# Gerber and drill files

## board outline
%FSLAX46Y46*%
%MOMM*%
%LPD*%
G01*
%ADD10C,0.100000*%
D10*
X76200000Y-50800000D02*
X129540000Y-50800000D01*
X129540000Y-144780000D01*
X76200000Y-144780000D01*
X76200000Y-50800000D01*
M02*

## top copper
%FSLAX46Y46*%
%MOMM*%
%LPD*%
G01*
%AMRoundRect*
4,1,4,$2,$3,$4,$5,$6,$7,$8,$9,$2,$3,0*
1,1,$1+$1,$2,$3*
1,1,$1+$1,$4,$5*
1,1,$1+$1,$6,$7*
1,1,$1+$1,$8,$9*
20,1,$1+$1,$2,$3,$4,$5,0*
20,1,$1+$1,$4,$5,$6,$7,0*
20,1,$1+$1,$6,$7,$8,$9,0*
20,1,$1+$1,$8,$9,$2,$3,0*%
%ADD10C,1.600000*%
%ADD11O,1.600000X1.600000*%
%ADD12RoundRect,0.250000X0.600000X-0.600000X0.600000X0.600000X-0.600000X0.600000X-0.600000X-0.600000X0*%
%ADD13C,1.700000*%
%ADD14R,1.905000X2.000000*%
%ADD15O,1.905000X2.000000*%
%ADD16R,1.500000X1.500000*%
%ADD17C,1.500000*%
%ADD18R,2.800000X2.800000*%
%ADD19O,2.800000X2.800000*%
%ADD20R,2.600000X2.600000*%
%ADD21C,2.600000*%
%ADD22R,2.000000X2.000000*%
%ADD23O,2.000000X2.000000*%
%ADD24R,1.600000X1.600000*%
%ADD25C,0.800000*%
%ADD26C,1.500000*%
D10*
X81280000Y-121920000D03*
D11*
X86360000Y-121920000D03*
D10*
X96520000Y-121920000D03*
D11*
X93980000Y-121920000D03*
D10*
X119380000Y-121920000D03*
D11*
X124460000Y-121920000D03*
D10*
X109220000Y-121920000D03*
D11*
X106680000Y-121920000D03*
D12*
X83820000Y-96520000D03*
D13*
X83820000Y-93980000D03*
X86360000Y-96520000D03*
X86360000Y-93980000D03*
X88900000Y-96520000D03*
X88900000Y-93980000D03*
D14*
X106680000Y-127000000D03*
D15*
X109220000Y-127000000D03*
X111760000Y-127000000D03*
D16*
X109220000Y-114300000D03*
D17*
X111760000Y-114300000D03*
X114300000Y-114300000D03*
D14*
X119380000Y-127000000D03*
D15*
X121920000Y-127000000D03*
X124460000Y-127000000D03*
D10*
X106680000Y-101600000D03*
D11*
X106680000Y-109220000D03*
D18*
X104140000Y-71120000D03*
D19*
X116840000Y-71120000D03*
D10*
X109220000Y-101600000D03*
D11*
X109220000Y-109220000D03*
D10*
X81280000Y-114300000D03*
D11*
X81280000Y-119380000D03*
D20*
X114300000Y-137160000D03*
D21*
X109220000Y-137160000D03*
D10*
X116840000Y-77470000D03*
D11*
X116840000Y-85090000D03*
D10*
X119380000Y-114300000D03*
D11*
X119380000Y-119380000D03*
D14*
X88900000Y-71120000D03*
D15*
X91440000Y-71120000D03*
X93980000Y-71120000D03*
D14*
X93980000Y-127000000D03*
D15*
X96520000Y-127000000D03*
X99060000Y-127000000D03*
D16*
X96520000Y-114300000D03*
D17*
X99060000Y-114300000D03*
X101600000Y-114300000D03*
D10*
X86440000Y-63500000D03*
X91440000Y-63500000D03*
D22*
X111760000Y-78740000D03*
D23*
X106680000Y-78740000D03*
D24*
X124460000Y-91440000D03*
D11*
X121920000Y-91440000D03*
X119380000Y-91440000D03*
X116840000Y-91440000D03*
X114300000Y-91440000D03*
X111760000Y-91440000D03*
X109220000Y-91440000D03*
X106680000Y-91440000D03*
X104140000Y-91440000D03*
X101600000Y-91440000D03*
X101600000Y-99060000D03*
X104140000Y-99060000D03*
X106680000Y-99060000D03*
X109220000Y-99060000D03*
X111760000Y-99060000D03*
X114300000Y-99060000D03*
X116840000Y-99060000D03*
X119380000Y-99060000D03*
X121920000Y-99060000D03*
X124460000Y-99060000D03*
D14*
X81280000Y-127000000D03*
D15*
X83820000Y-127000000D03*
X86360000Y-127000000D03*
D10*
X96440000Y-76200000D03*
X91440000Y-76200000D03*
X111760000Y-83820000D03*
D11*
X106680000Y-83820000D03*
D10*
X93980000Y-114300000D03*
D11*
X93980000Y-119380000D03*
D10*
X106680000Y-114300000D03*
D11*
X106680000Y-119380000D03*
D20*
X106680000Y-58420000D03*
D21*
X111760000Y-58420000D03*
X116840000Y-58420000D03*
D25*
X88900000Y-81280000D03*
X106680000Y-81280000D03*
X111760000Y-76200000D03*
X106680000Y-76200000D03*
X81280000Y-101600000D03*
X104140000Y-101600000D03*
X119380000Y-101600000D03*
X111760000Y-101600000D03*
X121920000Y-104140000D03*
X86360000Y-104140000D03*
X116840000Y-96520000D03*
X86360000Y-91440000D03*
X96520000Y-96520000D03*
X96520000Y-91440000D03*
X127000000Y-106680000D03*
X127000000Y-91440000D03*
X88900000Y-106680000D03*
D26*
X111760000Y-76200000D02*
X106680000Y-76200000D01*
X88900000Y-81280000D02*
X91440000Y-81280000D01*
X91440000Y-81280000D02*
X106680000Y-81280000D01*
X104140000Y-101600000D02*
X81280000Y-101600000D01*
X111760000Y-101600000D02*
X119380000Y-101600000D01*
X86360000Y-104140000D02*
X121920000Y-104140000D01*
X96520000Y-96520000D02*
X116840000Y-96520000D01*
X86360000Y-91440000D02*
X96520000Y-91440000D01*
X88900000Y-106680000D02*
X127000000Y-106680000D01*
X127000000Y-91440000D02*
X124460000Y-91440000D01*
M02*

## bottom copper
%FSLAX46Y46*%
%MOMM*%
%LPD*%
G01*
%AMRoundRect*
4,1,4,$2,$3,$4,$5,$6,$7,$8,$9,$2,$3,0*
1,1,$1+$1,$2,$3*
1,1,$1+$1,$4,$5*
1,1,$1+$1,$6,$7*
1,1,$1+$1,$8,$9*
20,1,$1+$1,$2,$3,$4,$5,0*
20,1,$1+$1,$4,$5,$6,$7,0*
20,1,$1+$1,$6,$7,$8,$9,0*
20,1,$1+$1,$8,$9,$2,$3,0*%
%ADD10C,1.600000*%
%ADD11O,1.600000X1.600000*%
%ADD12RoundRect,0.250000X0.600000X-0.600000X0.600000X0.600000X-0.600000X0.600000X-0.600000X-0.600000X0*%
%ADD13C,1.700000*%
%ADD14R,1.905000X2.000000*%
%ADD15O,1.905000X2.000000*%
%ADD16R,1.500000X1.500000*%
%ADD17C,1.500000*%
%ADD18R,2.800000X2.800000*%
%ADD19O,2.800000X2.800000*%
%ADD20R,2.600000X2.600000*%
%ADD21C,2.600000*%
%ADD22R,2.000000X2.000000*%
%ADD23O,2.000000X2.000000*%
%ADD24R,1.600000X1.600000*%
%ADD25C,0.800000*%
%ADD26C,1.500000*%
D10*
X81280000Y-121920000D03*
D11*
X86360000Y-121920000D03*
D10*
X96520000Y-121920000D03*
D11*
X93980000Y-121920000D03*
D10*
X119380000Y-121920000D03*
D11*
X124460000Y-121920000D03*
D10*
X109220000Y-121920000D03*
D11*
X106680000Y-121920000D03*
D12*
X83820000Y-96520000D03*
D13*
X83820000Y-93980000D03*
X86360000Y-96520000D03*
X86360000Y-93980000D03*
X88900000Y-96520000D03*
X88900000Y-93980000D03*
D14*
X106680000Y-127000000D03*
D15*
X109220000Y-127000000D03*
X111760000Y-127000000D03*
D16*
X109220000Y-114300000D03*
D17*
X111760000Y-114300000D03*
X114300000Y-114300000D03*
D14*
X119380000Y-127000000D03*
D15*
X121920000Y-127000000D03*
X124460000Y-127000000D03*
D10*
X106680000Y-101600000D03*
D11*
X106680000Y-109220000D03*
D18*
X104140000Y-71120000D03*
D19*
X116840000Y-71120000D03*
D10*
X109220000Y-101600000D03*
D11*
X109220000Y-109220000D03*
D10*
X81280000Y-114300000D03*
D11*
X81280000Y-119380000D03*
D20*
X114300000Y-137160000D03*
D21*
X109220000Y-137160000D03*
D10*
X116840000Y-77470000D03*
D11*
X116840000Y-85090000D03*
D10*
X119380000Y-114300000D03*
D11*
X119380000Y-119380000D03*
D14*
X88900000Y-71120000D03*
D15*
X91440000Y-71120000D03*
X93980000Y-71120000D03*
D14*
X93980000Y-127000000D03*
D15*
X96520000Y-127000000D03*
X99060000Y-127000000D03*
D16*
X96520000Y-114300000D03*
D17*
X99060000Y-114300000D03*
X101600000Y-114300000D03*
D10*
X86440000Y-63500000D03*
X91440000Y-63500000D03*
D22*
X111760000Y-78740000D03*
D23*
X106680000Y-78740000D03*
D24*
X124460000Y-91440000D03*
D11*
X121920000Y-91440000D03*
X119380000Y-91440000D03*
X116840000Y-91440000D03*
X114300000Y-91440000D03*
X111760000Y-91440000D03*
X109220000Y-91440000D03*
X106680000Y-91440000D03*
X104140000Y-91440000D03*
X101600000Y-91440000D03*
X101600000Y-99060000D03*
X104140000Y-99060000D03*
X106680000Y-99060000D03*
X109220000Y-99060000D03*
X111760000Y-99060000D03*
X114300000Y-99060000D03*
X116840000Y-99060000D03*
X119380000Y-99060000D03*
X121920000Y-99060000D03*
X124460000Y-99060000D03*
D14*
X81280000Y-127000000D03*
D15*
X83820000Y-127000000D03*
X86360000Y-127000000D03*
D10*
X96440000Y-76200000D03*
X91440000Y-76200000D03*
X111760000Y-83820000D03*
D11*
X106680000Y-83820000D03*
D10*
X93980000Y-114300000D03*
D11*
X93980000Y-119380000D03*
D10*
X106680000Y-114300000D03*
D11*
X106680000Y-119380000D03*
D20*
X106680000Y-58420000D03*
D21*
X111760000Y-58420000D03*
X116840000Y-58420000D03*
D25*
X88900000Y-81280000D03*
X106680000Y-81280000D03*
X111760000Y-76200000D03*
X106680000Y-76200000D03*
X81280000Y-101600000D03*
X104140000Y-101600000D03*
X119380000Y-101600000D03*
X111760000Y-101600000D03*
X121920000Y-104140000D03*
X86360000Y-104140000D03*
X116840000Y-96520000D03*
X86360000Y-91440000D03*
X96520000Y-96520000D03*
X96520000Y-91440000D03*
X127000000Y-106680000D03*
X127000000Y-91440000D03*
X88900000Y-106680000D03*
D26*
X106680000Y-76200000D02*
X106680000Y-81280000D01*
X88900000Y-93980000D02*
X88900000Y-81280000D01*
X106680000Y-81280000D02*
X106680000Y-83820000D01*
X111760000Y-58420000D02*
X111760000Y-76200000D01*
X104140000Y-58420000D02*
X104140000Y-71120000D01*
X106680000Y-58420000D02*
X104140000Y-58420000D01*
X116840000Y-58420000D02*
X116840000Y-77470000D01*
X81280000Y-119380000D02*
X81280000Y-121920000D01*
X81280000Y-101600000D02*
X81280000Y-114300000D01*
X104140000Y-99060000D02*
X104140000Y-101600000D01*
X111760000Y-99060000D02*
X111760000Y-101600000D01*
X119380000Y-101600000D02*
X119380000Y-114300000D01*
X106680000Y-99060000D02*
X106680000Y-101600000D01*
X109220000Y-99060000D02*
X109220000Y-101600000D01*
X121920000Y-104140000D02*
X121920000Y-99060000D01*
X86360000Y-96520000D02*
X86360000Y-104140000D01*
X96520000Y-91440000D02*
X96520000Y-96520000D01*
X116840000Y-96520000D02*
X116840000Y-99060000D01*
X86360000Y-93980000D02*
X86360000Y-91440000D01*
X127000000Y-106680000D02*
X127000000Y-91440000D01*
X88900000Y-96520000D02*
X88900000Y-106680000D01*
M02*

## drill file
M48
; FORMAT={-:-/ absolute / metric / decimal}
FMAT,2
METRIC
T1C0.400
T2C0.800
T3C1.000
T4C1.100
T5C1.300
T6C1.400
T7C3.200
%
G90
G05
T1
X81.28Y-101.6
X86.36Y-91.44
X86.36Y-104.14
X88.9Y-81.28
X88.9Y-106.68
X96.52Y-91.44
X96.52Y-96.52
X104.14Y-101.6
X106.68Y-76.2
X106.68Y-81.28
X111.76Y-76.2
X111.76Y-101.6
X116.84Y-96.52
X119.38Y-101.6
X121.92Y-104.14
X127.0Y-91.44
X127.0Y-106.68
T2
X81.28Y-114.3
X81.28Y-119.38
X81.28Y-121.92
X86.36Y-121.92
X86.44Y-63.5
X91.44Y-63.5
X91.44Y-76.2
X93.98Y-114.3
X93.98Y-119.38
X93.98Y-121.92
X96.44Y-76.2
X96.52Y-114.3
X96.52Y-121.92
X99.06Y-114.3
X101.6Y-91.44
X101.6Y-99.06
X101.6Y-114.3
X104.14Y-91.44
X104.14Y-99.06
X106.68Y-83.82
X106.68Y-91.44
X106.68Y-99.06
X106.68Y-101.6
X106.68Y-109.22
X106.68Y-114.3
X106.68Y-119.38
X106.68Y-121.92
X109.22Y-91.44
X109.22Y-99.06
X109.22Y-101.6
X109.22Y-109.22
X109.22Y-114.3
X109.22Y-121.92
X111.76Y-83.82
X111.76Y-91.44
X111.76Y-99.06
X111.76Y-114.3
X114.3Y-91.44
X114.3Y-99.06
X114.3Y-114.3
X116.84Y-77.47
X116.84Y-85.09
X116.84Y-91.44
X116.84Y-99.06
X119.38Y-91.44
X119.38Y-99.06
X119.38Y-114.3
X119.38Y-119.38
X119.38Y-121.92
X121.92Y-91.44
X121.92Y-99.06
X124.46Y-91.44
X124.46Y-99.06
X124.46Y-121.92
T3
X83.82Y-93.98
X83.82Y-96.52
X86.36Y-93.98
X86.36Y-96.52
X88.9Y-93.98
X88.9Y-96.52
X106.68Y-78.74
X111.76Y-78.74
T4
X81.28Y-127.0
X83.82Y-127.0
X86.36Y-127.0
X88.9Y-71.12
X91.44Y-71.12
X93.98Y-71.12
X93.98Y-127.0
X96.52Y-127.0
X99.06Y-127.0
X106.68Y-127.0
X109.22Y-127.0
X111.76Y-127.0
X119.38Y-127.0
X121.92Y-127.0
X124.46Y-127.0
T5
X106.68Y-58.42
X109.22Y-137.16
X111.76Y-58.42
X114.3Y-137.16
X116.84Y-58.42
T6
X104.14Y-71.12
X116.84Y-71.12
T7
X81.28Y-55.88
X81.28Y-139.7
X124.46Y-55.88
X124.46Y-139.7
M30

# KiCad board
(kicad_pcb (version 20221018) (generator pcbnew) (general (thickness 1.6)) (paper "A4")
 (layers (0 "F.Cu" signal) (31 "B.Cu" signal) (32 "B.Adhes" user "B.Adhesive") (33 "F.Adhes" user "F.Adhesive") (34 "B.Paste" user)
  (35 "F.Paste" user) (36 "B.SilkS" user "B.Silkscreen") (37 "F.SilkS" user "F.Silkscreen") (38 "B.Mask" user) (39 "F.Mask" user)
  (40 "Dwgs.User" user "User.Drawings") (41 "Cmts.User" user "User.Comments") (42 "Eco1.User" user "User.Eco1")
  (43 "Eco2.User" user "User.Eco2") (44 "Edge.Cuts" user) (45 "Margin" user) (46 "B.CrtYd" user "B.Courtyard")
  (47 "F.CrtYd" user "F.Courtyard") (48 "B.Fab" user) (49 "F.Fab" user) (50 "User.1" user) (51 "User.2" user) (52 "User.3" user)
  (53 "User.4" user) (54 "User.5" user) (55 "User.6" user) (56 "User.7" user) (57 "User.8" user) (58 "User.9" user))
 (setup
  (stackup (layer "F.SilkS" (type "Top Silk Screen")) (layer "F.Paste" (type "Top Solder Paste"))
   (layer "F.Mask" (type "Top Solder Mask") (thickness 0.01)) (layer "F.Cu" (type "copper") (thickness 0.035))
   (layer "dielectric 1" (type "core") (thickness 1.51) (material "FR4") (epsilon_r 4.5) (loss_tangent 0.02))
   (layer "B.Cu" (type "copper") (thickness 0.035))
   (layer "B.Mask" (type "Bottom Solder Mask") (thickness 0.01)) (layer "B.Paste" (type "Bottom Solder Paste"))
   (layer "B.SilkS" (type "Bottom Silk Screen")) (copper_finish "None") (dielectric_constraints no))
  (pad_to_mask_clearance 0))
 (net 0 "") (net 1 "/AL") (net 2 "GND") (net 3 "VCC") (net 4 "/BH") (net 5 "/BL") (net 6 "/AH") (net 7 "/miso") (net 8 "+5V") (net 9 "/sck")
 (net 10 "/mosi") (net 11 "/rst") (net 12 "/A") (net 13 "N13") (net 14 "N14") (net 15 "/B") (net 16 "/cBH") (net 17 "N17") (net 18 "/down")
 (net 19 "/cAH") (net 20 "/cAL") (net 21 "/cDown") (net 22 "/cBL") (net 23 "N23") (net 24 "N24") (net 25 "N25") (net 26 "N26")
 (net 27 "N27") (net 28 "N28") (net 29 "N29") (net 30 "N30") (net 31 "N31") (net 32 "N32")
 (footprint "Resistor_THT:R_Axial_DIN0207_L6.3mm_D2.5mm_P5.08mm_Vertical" (layer "F.Cu") (at 81.28 121.92)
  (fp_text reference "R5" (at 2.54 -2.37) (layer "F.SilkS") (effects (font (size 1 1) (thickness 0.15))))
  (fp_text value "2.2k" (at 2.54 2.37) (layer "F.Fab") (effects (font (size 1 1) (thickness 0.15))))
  (pad "1" thru_hole circle (at 0 0) (size 1.6 1.6) (drill 0.8) (layers "*.Cu" "*.Mask") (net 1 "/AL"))
  (pad "2" thru_hole oval (at 5.08 0) (size 1.6 1.6) (drill 0.8) (layers "*.Cu" "*.Mask") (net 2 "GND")))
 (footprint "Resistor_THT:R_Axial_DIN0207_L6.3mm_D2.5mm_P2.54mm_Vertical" (layer "F.Cu") (at 96.52 121.92 180)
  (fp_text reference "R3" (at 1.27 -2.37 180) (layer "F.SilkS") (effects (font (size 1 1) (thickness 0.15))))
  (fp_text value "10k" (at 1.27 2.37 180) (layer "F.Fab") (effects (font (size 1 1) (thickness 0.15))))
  (pad "1" thru_hole circle (at 0 0 180) (size 1.6 1.6) (drill 0.8) (layers "*.Cu" "*.Mask") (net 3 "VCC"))
  (pad "2" thru_hole oval (at 2.54 0 180) (size 1.6 1.6) (drill 0.8) (layers "*.Cu" "*.Mask") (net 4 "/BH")))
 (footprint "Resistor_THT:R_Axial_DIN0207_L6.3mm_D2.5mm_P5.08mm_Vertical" (layer "F.Cu") (at 119.38 121.92)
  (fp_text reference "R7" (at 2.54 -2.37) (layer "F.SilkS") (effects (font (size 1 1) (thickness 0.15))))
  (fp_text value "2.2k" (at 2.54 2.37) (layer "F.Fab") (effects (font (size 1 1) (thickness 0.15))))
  (pad "1" thru_hole circle (at 0 0) (size 1.6 1.6) (drill 0.8) (layers "*.Cu" "*.Mask") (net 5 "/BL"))
  (pad "2" thru_hole oval (at 5.08 0) (size 1.6 1.6) (drill 0.8) (layers "*.Cu" "*.Mask") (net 2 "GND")))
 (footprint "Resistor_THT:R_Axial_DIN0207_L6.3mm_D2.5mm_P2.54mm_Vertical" (layer "F.Cu") (at 109.22 121.92 180)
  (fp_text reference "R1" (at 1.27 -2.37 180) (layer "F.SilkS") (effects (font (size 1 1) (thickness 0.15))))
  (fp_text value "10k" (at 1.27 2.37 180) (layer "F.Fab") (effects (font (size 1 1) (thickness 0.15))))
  (pad "1" thru_hole circle (at 0 0 180) (size 1.6 1.6) (drill 0.8) (layers "*.Cu" "*.Mask") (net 3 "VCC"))
  (pad "2" thru_hole oval (at 2.54 0 180) (size 1.6 1.6) (drill 0.8) (layers "*.Cu" "*.Mask") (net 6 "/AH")))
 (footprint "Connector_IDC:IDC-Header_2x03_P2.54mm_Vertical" (layer "F.Cu") (at 83.82 96.52 90)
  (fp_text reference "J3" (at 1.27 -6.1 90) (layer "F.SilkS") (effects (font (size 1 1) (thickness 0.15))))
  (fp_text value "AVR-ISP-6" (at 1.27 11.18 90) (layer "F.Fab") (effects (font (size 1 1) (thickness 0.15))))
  (pad "1" thru_hole roundrect (at 0 0 90) (size 1.7 1.7) (drill 1) (layers "*.Cu" "*.Mask") (roundrect_rratio 0.147059) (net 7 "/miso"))
  (pad "2" thru_hole circle (at 2.54 0 90) (size 1.7 1.7) (drill 1) (layers "*.Cu" "*.Mask") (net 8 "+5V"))
  (pad "3" thru_hole circle (at 0 2.54 90) (size 1.7 1.7) (drill 1) (layers "*.Cu" "*.Mask") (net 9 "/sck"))
  (pad "4" thru_hole circle (at 2.54 2.54 90) (size 1.7 1.7) (drill 1) (layers "*.Cu" "*.Mask") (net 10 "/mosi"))
  (pad "5" thru_hole circle (at 0 5.08 90) (size 1.7 1.7) (drill 1) (layers "*.Cu" "*.Mask") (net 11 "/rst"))
  (pad "6" thru_hole circle (at 2.54 5.08 90) (size 1.7 1.7) (drill 1) (layers "*.Cu" "*.Mask") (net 2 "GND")))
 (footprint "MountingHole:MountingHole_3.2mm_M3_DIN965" (layer "F.Cu") (at 81.28 139.7)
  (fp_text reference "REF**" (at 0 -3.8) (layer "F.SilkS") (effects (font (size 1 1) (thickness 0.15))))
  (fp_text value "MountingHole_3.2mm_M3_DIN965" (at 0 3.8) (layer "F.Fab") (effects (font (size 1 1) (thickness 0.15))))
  (pad "" np_thru_hole circle (at 0 0) (size 3.2 3.2) (drill 3.2) (layers "*.Cu" "*.Mask")))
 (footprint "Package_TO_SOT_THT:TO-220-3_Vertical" (layer "F.Cu") (at 106.68 127)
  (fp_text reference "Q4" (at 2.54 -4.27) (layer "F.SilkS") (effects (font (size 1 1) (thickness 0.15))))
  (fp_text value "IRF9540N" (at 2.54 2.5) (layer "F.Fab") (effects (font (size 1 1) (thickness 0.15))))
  (pad "1" thru_hole rect (at 0 0) (size 1.905 2) (drill 1.1) (layers "*.Cu" "*.Mask") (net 6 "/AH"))
  (pad "2" thru_hole oval (at 2.54 0) (size 1.905 2) (drill 1.1) (layers "*.Cu" "*.Mask") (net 3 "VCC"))
  (pad "3" thru_hole oval (at 5.08 0) (size 1.905 2) (drill 1.1) (layers "*.Cu" "*.Mask") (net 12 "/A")))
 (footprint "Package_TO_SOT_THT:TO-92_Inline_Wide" (layer "F.Cu") (at 109.22 114.3)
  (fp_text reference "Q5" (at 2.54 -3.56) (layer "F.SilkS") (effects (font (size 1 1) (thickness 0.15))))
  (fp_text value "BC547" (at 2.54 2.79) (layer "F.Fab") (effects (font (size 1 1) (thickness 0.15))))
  (pad "1" thru_hole rect (at 0 0) (size 1.5 1.5) (drill 0.8) (layers "*.Cu" "*.Mask") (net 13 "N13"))
  (pad "2" thru_hole circle (at 2.54 0) (size 1.5 1.5) (drill 0.8) (layers "*.Cu" "*.Mask") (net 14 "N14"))
  (pad "3" thru_hole circle (at 5.08 0) (size 1.5 1.5) (drill 0.8) (layers "*.Cu" "*.Mask") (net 2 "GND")))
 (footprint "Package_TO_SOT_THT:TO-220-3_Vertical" (layer "F.Cu") (at 119.38 127)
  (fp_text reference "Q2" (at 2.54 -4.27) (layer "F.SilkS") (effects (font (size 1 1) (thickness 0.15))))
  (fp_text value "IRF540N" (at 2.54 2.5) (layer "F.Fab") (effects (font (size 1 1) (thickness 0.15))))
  (pad "1" thru_hole rect (at 0 0) (size 1.905 2) (drill 1.1) (layers "*.Cu" "*.Mask") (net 5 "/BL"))
  (pad "2" thru_hole oval (at 2.54 0) (size 1.905 2) (drill 1.1) (layers "*.Cu" "*.Mask") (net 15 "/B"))
  (pad "3" thru_hole oval (at 5.08 0) (size 1.905 2) (drill 1.1) (layers "*.Cu" "*.Mask") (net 2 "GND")))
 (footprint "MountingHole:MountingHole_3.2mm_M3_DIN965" (layer "F.Cu") (at 124.46 55.88)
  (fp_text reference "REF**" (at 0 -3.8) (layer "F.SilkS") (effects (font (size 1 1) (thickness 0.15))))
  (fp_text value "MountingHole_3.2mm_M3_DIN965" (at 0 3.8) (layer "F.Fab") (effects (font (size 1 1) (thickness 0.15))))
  (pad "" np_thru_hole circle (at 0 0) (size 3.2 3.2) (drill 3.2) (layers "*.Cu" "*.Mask")))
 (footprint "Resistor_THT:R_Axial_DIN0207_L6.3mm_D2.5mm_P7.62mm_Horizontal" (layer "F.Cu") (at 106.68 101.6 -90)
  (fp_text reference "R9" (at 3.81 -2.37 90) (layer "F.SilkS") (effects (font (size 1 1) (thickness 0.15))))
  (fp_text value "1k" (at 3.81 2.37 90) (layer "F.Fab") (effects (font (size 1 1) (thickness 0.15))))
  (pad "1" thru_hole circle (at 0 0 270) (size 1.6 1.6) (drill 0.8) (layers "*.Cu" "*.Mask") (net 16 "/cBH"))
  (pad "2" thru_hole oval (at 7.62 0 270) (size 1.6 1.6) (drill 0.8) (layers "*.Cu" "*.Mask") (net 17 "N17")))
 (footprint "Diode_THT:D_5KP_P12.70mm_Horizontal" (layer "F.Cu") (at 104.14 71.12)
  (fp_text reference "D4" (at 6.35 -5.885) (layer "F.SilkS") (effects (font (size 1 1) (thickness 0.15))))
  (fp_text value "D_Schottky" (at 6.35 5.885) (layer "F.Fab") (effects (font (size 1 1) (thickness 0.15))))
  (pad "1" thru_hole rect (at 0 0) (size 2.8 2.8) (drill 1.4) (layers "*.Cu" "*.Mask") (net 3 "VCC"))
  (pad "2" thru_hole oval (at 12.7 0) (size 2.8 2.8) (drill 1.4) (layers "*.Cu" "*.Mask") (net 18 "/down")))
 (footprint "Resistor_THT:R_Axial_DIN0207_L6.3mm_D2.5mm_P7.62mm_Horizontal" (layer "F.Cu") (at 109.22 101.6 -90)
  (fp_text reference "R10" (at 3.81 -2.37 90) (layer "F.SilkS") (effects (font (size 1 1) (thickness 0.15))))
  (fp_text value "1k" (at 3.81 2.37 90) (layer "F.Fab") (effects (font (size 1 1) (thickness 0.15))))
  (pad "1" thru_hole circle (at 0 0 270) (size 1.6 1.6) (drill 0.8) (layers "*.Cu" "*.Mask") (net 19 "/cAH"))
  (pad "2" thru_hole oval (at 7.62 0 270) (size 1.6 1.6) (drill 0.8) (layers "*.Cu" "*.Mask") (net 14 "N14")))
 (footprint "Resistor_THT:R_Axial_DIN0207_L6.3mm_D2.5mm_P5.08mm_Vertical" (layer "F.Cu") (at 81.28 114.3 -90)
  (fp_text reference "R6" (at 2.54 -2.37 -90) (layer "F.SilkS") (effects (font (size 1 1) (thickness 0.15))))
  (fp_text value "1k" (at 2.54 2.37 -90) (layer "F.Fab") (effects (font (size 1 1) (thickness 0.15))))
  (pad "1" thru_hole circle (at 0 0 270) (size 1.6 1.6) (drill 0.8) (layers "*.Cu" "*.Mask") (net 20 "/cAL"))
  (pad "2" thru_hole oval (at 5.08 0 270) (size 1.6 1.6) (drill 0.8) (layers "*.Cu" "*.Mask") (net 1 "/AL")))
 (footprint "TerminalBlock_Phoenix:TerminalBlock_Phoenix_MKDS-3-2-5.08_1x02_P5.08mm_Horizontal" (layer "F.Cu") (at 114.3 137.16 180)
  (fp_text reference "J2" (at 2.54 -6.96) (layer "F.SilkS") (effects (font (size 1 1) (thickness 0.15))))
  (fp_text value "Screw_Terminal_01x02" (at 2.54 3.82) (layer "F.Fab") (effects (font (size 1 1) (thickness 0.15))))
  (pad "1" thru_hole rect (at 0 0 180) (size 2.6 2.6) (drill 1.3) (layers "*.Cu" "*.Mask") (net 12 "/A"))
  (pad "2" thru_hole circle (at 5.08 0 180) (size 2.6 2.6) (drill 1.3) (layers "*.Cu" "*.Mask") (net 15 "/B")))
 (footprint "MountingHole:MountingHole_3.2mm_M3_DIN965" (layer "F.Cu") (at 124.46 139.7)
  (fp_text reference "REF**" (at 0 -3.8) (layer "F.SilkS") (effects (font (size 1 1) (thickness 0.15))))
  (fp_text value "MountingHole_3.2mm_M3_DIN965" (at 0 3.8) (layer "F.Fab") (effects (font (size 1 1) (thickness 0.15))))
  (pad "" np_thru_hole circle (at 0 0) (size 3.2 3.2) (drill 3.2) (layers "*.Cu" "*.Mask")))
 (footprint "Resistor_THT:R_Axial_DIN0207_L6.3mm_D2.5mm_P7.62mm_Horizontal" (layer "F.Cu") (at 116.84 77.47 -90)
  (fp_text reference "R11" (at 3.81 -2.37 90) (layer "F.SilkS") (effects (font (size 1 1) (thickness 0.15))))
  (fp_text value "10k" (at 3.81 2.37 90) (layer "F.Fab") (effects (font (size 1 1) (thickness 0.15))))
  (pad "1" thru_hole circle (at 0 0 270) (size 1.6 1.6) (drill 0.8) (layers "*.Cu" "*.Mask") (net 18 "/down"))
  (pad "2" thru_hole oval (at 7.62 0 270) (size 1.6 1.6) (drill 0.8) (layers "*.Cu" "*.Mask") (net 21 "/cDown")))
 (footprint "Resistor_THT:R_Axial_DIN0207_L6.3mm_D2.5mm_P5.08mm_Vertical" (layer "F.Cu") (at 119.38 114.3 -90)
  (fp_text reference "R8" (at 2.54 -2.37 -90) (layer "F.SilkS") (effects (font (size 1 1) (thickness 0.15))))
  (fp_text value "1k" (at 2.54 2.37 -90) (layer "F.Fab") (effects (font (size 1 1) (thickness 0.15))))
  (pad "1" thru_hole circle (at 0 0 270) (size 1.6 1.6) (drill 0.8) (layers "*.Cu" "*.Mask") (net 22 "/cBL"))
  (pad "2" thru_hole oval (at 5.08 0 270) (size 1.6 1.6) (drill 0.8) (layers "*.Cu" "*.Mask") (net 5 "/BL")))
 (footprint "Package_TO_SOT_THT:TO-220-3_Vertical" (layer "F.Cu") (at 88.9 71.12)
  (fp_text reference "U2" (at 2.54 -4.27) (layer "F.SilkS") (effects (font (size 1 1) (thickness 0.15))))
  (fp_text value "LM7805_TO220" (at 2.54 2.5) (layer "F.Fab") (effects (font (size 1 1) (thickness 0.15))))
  (pad "1" thru_hole rect (at 0 0) (size 1.905 2) (drill 1.1) (layers "*.Cu" "*.Mask") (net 3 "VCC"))
  (pad "2" thru_hole oval (at 2.54 0) (size 1.905 2) (drill 1.1) (layers "*.Cu" "*.Mask") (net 2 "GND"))
  (pad "3" thru_hole oval (at 5.08 0) (size 1.905 2) (drill 1.1) (layers "*.Cu" "*.Mask") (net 8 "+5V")))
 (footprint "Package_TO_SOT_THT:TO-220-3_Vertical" (layer "F.Cu") (at 93.98 127)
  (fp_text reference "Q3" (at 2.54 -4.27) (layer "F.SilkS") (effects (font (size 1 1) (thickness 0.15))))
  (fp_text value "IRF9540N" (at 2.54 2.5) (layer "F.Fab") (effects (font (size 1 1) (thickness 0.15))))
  (pad "1" thru_hole rect (at 0 0) (size 1.905 2) (drill 1.1) (layers "*.Cu" "*.Mask") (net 4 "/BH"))
  (pad "2" thru_hole oval (at 2.54 0) (size 1.905 2) (drill 1.1) (layers "*.Cu" "*.Mask") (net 3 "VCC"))
  (pad "3" thru_hole oval (at 5.08 0) (size 1.905 2) (drill 1.1) (layers "*.Cu" "*.Mask") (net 15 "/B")))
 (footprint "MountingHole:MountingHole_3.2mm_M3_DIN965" (layer "F.Cu") (at 81.28 55.88)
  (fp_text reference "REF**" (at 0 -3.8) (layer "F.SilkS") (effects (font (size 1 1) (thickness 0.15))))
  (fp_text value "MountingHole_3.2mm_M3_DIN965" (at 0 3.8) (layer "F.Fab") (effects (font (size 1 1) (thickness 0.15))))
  (pad "" np_thru_hole circle (at 0 0) (size 3.2 3.2) (drill 3.2) (layers "*.Cu" "*.Mask")))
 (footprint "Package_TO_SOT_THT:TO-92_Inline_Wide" (layer "F.Cu") (at 96.52 114.3)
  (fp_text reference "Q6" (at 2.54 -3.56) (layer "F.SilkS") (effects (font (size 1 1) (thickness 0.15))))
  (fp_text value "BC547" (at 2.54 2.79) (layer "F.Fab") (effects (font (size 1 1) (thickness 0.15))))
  (pad "1" thru_hole rect (at 0 0) (size 1.5 1.5) (drill 0.8) (layers "*.Cu" "*.Mask") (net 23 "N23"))
  (pad "2" thru_hole circle (at 2.54 0) (size 1.5 1.5) (drill 0.8) (layers "*.Cu" "*.Mask") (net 17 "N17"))
  (pad "3" thru_hole circle (at 5.08 0) (size 1.5 1.5) (drill 0.8) (layers "*.Cu" "*.Mask") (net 2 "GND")))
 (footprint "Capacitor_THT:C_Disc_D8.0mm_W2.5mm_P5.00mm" (layer "F.Cu") (at 86.44 63.5)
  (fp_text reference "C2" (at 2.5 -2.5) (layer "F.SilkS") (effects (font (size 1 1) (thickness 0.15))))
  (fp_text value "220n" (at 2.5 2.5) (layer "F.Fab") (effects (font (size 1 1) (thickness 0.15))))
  (pad "1" thru_hole circle (at 0 0) (size 1.6 1.6) (drill 0.8) (layers "*.Cu" "*.Mask") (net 3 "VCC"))
  (pad "2" thru_hole circle (at 5 0) (size 1.6 1.6) (drill 0.8) (layers "*.Cu" "*.Mask") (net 2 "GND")))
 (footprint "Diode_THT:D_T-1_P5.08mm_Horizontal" (layer "F.Cu") (at 111.76 78.74 180)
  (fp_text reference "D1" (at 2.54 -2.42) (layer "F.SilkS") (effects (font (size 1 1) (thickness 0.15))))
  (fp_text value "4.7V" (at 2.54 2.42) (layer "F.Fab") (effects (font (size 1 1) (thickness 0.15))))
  (pad "1" thru_hole rect (at 0 0 180) (size 2 2) (drill 1) (layers "*.Cu" "*.Mask") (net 21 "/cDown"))
  (pad "2" thru_hole oval (at 5.08 0 180) (size 2 2) (drill 1) (layers "*.Cu" "*.Mask") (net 2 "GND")))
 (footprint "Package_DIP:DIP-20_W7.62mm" (layer "F.Cu") (at 124.46 91.44 -90)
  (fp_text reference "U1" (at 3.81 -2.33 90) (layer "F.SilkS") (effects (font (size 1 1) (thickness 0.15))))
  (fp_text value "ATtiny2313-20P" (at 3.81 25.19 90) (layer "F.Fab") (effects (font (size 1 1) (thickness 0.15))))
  (pad "1" thru_hole rect (at 0 0 270) (size 1.6 1.6) (drill 0.8) (layers "*.Cu" "*.Mask") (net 11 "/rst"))
  (pad "2" thru_hole oval (at 0 2.54 270) (size 1.6 1.6) (drill 0.8) (layers "*.Cu" "*.Mask") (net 21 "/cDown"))
  (pad "3" thru_hole oval (at 0 5.08 270) (size 1.6 1.6) (drill 0.8) (layers "*.Cu" "*.Mask") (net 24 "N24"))
  (pad "4" thru_hole oval (at 0 7.62 270) (size 1.6 1.6) (drill 0.8) (layers "*.Cu" "*.Mask") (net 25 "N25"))
  (pad "5" thru_hole oval (at 0 10.16 270) (size 1.6 1.6) (drill 0.8) (layers "*.Cu" "*.Mask") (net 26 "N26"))
  (pad "6" thru_hole oval (at 0 12.7 270) (size 1.6 1.6) (drill 0.8) (layers "*.Cu" "*.Mask") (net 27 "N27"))
  (pad "7" thru_hole oval (at 0 15.24 270) (size 1.6 1.6) (drill 0.8) (layers "*.Cu" "*.Mask") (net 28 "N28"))
  (pad "8" thru_hole oval (at 0 17.78 270) (size 1.6 1.6) (drill 0.8) (layers "*.Cu" "*.Mask") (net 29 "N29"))
  (pad "9" thru_hole oval (at 0 20.32 270) (size 1.6 1.6) (drill 0.8) (layers "*.Cu" "*.Mask") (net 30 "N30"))
  (pad "10" thru_hole oval (at 0 22.86 270) (size 1.6 1.6) (drill 0.8) (layers "*.Cu" "*.Mask") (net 2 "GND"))
  (pad "11" thru_hole oval (at 7.62 22.86 270) (size 1.6 1.6) (drill 0.8) (layers "*.Cu" "*.Mask") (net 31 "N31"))
  (pad "12" thru_hole oval (at 7.62 20.32 270) (size 1.6 1.6) (drill 0.8) (layers "*.Cu" "*.Mask") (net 20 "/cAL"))
  (pad "13" thru_hole oval (at 7.62 17.78 270) (size 1.6 1.6) (drill 0.8) (layers "*.Cu" "*.Mask") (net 16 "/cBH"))
  (pad "14" thru_hole oval (at 7.62 15.24 270) (size 1.6 1.6) (drill 0.8) (layers "*.Cu" "*.Mask") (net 19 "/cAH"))
  (pad "15" thru_hole oval (at 7.62 12.7 270) (size 1.6 1.6) (drill 0.8) (layers "*.Cu" "*.Mask") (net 22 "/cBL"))
  (pad "16" thru_hole oval (at 7.62 10.16 270) (size 1.6 1.6) (drill 0.8) (layers "*.Cu" "*.Mask") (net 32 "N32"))
  (pad "17" thru_hole oval (at 7.62 7.62 270) (size 1.6 1.6) (drill 0.8) (layers "*.Cu" "*.Mask") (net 10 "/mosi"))
  (pad "18" thru_hole oval (at 7.62 5.08 270) (size 1.6 1.6) (drill 0.8) (layers "*.Cu" "*.Mask") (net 7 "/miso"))
  (pad "19" thru_hole oval (at 7.62 2.54 270) (size 1.6 1.6) (drill 0.8) (layers "*.Cu" "*.Mask") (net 9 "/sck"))
  (pad "20" thru_hole oval (at 7.62 0 270) (size 1.6 1.6) (drill 0.8) (layers "*.Cu" "*.Mask") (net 8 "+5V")))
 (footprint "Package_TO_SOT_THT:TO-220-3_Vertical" (layer "F.Cu") (at 81.28 127)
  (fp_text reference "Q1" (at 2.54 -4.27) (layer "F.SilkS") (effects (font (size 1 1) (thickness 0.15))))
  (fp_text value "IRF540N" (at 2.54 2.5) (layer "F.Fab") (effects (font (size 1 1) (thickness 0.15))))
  (pad "1" thru_hole rect (at 0 0) (size 1.905 2) (drill 1.1) (layers "*.Cu" "*.Mask") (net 1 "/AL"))
  (pad "2" thru_hole oval (at 2.54 0) (size 1.905 2) (drill 1.1) (layers "*.Cu" "*.Mask") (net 12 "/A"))
  (pad "3" thru_hole oval (at 5.08 0) (size 1.905 2) (drill 1.1) (layers "*.Cu" "*.Mask") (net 2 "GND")))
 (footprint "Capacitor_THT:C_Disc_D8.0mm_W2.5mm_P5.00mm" (layer "F.Cu") (at 96.44 76.2 180)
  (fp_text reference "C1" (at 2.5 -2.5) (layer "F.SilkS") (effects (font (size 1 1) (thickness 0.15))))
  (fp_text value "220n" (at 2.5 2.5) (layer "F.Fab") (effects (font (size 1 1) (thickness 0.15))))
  (pad "1" thru_hole circle (at 0 0 180) (size 1.6 1.6) (drill 0.8) (layers "*.Cu" "*.Mask") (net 8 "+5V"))
  (pad "2" thru_hole circle (at 5 0 180) (size 1.6 1.6) (drill 0.8) (layers "*.Cu" "*.Mask") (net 2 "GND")))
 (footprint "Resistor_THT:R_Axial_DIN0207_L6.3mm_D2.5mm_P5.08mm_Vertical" (layer "F.Cu") (at 111.76 83.82 180)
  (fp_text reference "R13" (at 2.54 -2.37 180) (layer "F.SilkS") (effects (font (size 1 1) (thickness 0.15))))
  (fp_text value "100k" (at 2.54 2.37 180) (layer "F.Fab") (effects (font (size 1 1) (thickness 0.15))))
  (pad "1" thru_hole circle (at 0 0 180) (size 1.6 1.6) (drill 0.8) (layers "*.Cu" "*.Mask") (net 21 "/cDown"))
  (pad "2" thru_hole oval (at 5.08 0 180) (size 1.6 1.6) (drill 0.8) (layers "*.Cu" "*.Mask") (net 2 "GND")))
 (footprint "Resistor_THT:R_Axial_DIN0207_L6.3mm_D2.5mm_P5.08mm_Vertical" (layer "F.Cu") (at 93.98 114.3 -90)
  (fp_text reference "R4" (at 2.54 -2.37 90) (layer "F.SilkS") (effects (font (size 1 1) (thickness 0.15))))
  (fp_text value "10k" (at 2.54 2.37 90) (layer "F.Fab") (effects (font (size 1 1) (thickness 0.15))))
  (pad "1" thru_hole circle (at 0 0 270) (size 1.6 1.6) (drill 0.8) (layers "*.Cu" "*.Mask") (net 23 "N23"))
  (pad "2" thru_hole oval (at 5.08 0 270) (size 1.6 1.6) (drill 0.8) (layers "*.Cu" "*.Mask") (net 4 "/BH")))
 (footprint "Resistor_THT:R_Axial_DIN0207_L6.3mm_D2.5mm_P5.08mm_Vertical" (layer "F.Cu") (at 106.68 114.3 -90)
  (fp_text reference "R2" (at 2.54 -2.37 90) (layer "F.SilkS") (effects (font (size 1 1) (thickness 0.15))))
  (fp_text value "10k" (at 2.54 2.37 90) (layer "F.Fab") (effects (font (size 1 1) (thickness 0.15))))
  (pad "1" thru_hole circle (at 0 0 270) (size 1.6 1.6) (drill 0.8) (layers "*.Cu" "*.Mask") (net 13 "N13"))
  (pad "2" thru_hole oval (at 5.08 0 270) (size 1.6 1.6) (drill 0.8) (layers "*.Cu" "*.Mask") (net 6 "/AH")))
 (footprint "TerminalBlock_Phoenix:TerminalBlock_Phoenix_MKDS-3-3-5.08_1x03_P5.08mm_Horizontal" (layer "F.Cu") (at 106.68 58.42)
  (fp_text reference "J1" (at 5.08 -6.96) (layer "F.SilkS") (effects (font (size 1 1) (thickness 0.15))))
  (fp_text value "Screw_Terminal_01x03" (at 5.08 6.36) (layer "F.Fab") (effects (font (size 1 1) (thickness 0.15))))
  (pad "1" thru_hole rect (at 0 0) (size 2.6 2.6) (drill 1.3) (layers "*.Cu" "*.Mask") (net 3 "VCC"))
  (pad "2" thru_hole circle (at 5.08 0) (size 2.6 2.6) (drill 1.3) (layers "*.Cu" "*.Mask") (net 2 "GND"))
  (pad "3" thru_hole circle (at 10.16 0) (size 2.6 2.6) (drill 1.3) (layers "*.Cu" "*.Mask") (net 18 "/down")))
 (gr_rect (start 76.2 50.8) (end 129.54 144.78) (stroke (width 0.1) (type default)) (fill none) (layer "Edge.Cuts"))
 (segment (start 111.76 76.2) (end 106.68 76.2) (width 1.5) (layer "F.Cu") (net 2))
 (segment (start 88.9 81.28) (end 91.44 81.28) (width 1.5) (layer "F.Cu") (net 2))
 (segment (start 91.44 81.28) (end 106.68 81.28) (width 1.5) (layer "F.Cu") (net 2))
 (via (at 88.9 81.28) (size 0.8) (drill 0.4) (layers "F.Cu" "B.Cu") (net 2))
 (via (at 106.68 81.28) (size 0.8) (drill 0.4) (layers "F.Cu" "B.Cu") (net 2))
 (via (at 111.76 76.2) (size 0.8) (drill 0.4) (layers "F.Cu" "B.Cu") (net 2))
 (via (at 106.68 76.2) (size 0.8) (drill 0.4) (layers "F.Cu" "B.Cu") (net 2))
 (segment (start 106.68 76.2) (end 106.68 81.28) (width 1.5) (layer "B.Cu") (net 2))
 (segment (start 88.9 93.98) (end 88.9 81.28) (width 1.5) (layer "B.Cu") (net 2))
 (segment (start 106.68 81.28) (end 106.68 83.82) (width 1.5) (layer "B.Cu") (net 2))
 (segment (start 111.76 58.42) (end 111.76 76.2) (width 1.5) (layer "B.Cu") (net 2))
 (segment (start 104.14 58.42) (end 104.14 71.12) (width 1.5) (layer "B.Cu") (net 3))
 (segment (start 106.68 58.42) (end 104.14 58.42) (width 1.5) (layer "B.Cu") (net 3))
 (segment (start 116.84 58.42) (end 116.84 77.47) (width 1.5) (layer "B.Cu") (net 18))
 (segment (start 81.28 119.38) (end 81.28 121.92) (width 1.5) (layer "B.Cu") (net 1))
 (segment (start 104.14 101.6) (end 81.28 101.6) (width 1.5) (layer "F.Cu") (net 20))
 (via (at 81.28 101.6) (size 0.8) (drill 0.4) (layers "F.Cu" "B.Cu") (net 20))
 (via (at 104.14 101.6) (size 0.8) (drill 0.4) (layers "F.Cu" "B.Cu") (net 20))
 (segment (start 81.28 101.6) (end 81.28 114.3) (width 1.5) (layer "B.Cu") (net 20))
 (segment (start 104.14 99.06) (end 104.14 101.6) (width 1.5) (layer "B.Cu") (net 20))
 (segment (start 111.76 101.6) (end 119.38 101.6) (width 1.5) (layer "F.Cu") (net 22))
 (via (at 119.38 101.6) (size 0.8) (drill 0.4) (layers "F.Cu" "B.Cu") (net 22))
 (via (at 111.76 101.6) (size 0.8) (drill 0.4) (layers "F.Cu" "B.Cu") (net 22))
 (segment (start 111.76 99.06) (end 111.76 101.6) (width 1.5) (layer "B.Cu") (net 22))
 (segment (start 119.38 101.6) (end 119.38 114.3) (width 1.5) (layer "B.Cu") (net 22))
 (segment (start 106.68 99.06) (end 106.68 101.6) (width 1.5) (layer "B.Cu") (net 16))
 (segment (start 109.22 99.06) (end 109.22 101.6) (width 1.5) (layer "B.Cu") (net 19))
 (segment (start 86.36 104.14) (end 121.92 104.14) (width 1.5) (layer "F.Cu") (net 9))
 (via (at 121.92 104.14) (size 0.8) (drill 0.4) (layers "F.Cu" "B.Cu") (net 9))
 (via (at 86.36 104.14) (size 0.8) (drill 0.4) (layers "F.Cu" "B.Cu") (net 9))
 (segment (start 121.92 104.14) (end 121.92 99.06) (width 1.5) (layer "B.Cu") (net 9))
 (segment (start 86.36 96.52) (end 86.36 104.14) (width 1.5) (layer "B.Cu") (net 9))
 (segment (start 96.52 96.52) (end 116.84 96.52) (width 1.5) (layer "F.Cu") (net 10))
 (segment (start 86.36 91.44) (end 96.52 91.44) (width 1.5) (layer "F.Cu") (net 10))
 (via (at 116.84 96.52) (size 0.8) (drill 0.4) (layers "F.Cu" "B.Cu") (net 10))
 (via (at 86.36 91.44) (size 0.8) (drill 0.4) (layers "F.Cu" "B.Cu") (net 10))
 (via (at 96.52 96.52) (size 0.8) (drill 0.4) (layers "F.Cu" "B.Cu") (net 10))
 (via (at 96.52 91.44) (size 0.8) (drill 0.4) (layers "F.Cu" "B.Cu") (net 10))
 (segment (start 96.52 91.44) (end 96.52 96.52) (width 1.5) (layer "B.Cu") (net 10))
 (segment (start 116.84 96.52) (end 116.84 99.06) (width 1.5) (layer "B.Cu") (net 10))
 (segment (start 86.36 93.98) (end 86.36 91.44) (width 1.5) (layer "B.Cu") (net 10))
 (segment (start 88.9 106.68) (end 127 106.68) (width 1.5) (layer "F.Cu") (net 11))
 (segment (start 127 91.44) (end 124.46 91.44) (width 1.5) (layer "F.Cu") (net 11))
 (via (at 127 106.68) (size 0.8) (drill 0.4) (layers "F.Cu" "B.Cu") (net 11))
 (via (at 127 91.44) (size 0.8) (drill 0.4) (layers "F.Cu" "B.Cu") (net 11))
 (via (at 88.9 106.68) (size 0.8) (drill 0.4) (layers "F.Cu" "B.Cu") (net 11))
 (segment (start 127 106.68) (end 127 91.44) (width 1.5) (layer "B.Cu") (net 11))
 (segment (start 88.9 96.52) (end 88.9 106.68) (width 1.5) (layer "B.Cu") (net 11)))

